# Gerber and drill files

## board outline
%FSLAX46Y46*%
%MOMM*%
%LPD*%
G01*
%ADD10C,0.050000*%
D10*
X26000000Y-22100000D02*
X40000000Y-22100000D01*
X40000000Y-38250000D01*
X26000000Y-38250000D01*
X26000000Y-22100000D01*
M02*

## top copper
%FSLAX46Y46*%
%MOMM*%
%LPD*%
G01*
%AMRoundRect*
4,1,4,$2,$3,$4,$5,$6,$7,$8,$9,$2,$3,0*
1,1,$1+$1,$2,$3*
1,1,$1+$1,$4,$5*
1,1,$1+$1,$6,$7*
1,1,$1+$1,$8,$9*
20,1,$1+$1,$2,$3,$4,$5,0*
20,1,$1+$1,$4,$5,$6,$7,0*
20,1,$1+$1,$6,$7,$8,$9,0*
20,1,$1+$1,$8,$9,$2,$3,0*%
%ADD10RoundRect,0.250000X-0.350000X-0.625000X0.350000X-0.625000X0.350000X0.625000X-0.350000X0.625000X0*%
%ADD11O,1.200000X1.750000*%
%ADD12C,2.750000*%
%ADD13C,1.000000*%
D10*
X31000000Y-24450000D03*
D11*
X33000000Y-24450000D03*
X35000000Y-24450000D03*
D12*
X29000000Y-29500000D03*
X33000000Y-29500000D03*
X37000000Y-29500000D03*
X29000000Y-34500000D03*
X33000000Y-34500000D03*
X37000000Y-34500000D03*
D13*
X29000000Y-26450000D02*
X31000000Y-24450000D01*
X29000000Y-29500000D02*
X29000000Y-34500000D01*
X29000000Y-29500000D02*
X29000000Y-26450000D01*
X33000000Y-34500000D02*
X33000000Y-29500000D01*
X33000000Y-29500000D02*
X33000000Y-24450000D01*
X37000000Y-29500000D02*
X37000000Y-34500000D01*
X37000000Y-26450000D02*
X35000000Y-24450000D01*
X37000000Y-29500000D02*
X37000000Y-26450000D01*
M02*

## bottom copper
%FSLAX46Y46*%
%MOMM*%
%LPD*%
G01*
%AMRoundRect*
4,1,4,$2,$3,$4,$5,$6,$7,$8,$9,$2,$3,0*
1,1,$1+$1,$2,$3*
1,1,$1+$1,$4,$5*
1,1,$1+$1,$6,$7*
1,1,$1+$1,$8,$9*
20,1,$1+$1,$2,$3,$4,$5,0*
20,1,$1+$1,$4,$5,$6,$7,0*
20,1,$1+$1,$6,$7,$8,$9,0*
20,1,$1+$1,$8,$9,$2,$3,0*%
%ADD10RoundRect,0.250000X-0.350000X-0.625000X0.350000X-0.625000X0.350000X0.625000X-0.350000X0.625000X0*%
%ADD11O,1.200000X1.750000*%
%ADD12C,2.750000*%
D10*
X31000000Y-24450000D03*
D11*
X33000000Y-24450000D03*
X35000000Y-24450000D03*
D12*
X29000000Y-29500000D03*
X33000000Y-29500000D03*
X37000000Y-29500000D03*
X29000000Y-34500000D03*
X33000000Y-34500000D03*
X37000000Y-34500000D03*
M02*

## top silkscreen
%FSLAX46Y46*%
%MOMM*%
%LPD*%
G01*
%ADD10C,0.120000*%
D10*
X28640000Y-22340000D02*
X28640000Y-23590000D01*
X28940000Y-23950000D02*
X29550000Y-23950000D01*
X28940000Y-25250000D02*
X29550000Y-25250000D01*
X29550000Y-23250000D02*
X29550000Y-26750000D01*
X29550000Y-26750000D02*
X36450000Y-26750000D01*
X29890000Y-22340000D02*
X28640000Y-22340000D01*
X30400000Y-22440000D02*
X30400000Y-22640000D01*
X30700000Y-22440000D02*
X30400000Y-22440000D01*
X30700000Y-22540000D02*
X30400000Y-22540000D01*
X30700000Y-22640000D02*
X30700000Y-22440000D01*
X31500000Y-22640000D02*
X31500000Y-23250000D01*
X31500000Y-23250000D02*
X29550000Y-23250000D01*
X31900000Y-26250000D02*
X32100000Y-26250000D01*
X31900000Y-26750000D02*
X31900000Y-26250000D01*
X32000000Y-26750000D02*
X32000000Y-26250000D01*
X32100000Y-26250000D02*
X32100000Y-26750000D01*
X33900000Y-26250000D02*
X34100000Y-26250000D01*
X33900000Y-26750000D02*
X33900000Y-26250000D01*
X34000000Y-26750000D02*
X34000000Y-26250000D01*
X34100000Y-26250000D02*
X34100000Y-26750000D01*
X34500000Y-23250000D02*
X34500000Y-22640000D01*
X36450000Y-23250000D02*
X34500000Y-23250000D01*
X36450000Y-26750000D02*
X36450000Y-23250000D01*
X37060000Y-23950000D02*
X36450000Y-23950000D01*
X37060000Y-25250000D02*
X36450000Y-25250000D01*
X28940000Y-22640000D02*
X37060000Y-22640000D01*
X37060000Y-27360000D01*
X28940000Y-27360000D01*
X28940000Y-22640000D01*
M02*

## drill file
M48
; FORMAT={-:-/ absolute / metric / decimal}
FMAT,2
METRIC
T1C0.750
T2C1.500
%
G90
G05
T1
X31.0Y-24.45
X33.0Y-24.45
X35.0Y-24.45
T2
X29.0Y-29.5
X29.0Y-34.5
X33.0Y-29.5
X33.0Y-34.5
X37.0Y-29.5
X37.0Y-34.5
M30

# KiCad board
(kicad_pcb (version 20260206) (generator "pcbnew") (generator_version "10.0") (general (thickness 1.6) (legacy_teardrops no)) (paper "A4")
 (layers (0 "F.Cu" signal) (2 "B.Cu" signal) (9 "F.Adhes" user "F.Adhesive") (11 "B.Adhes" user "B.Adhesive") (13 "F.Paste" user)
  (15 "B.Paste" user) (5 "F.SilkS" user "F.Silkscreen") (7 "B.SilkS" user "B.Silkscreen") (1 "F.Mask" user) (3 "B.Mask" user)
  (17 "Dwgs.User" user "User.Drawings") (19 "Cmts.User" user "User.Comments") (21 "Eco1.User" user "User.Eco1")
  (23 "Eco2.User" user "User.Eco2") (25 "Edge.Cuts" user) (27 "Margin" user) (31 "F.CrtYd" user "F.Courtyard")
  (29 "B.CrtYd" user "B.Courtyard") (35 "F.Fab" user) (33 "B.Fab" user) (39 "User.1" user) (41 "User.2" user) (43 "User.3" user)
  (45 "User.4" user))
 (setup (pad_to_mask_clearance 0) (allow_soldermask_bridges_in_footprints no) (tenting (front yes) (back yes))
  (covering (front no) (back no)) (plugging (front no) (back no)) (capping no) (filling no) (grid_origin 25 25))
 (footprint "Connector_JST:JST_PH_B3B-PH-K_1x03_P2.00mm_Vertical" (layer "F.Cu") (at 31 24.45)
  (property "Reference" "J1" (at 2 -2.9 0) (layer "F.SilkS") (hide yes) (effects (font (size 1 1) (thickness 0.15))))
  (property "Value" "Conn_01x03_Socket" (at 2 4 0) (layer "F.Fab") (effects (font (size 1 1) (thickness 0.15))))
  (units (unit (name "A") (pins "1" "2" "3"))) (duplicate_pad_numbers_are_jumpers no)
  (fp_line (start -2.36 -2.11) (end -2.36 -0.86) (stroke (width 0.12) (type solid)) (layer "F.SilkS"))
  (fp_line (start -2.06 -0.5) (end -1.45 -0.5) (stroke (width 0.12) (type solid)) (layer "F.SilkS"))
  (fp_line (start -2.06 0.8) (end -1.45 0.8) (stroke (width 0.12) (type solid)) (layer "F.SilkS"))
  (fp_line (start -1.45 -1.2) (end -1.45 2.3) (stroke (width 0.12) (type solid)) (layer "F.SilkS"))
  (fp_line (start -1.45 2.3) (end 5.45 2.3) (stroke (width 0.12) (type solid)) (layer "F.SilkS"))
  (fp_line (start -1.11 -2.11) (end -2.36 -2.11) (stroke (width 0.12) (type solid)) (layer "F.SilkS"))
  (fp_line (start -0.6 -2.01) (end -0.6 -1.81) (stroke (width 0.12) (type solid)) (layer "F.SilkS"))
  (fp_line (start -0.3 -2.01) (end -0.6 -2.01) (stroke (width 0.12) (type solid)) (layer "F.SilkS"))
  (fp_line (start -0.3 -1.91) (end -0.6 -1.91) (stroke (width 0.12) (type solid)) (layer "F.SilkS"))
  (fp_line (start -0.3 -1.81) (end -0.3 -2.01) (stroke (width 0.12) (type solid)) (layer "F.SilkS"))
  (fp_line (start 0.5 -1.81) (end 0.5 -1.2) (stroke (width 0.12) (type solid)) (layer "F.SilkS"))
  (fp_line (start 0.5 -1.2) (end -1.45 -1.2) (stroke (width 0.12) (type solid)) (layer "F.SilkS"))
  (fp_line (start 0.9 1.8) (end 1.1 1.8) (stroke (width 0.12) (type solid)) (layer "F.SilkS"))
  (fp_line (start 0.9 2.3) (end 0.9 1.8) (stroke (width 0.12) (type solid)) (layer "F.SilkS"))
  (fp_line (start 1 2.3) (end 1 1.8) (stroke (width 0.12) (type solid)) (layer "F.SilkS"))
  (fp_line (start 1.1 1.8) (end 1.1 2.3) (stroke (width 0.12) (type solid)) (layer "F.SilkS"))
  (fp_line (start 2.9 1.8) (end 3.1 1.8) (stroke (width 0.12) (type solid)) (layer "F.SilkS"))
  (fp_line (start 2.9 2.3) (end 2.9 1.8) (stroke (width 0.12) (type solid)) (layer "F.SilkS"))
  (fp_line (start 3 2.3) (end 3 1.8) (stroke (width 0.12) (type solid)) (layer "F.SilkS"))
  (fp_line (start 3.1 1.8) (end 3.1 2.3) (stroke (width 0.12) (type solid)) (layer "F.SilkS"))
  (fp_line (start 3.5 -1.2) (end 3.5 -1.81) (stroke (width 0.12) (type solid)) (layer "F.SilkS"))
  (fp_line (start 5.45 -1.2) (end 3.5 -1.2) (stroke (width 0.12) (type solid)) (layer "F.SilkS"))
  (fp_line (start 5.45 2.3) (end 5.45 -1.2) (stroke (width 0.12) (type solid)) (layer "F.SilkS"))
  (fp_line (start 6.06 -0.5) (end 5.45 -0.5) (stroke (width 0.12) (type solid)) (layer "F.SilkS"))
  (fp_line (start 6.06 0.8) (end 5.45 0.8) (stroke (width 0.12) (type solid)) (layer "F.SilkS"))
  (fp_rect (start -2.06 -1.81) (end 6.06 2.91) (stroke (width 0.12) (type solid)) (fill no) (layer "F.SilkS"))
  (pad "1" thru_hole roundrect (at 0 0) (size 1.2 1.75) (drill 0.75) (layers "*.Cu" "*.Mask") (remove_unused_layers no)
   (roundrect_rratio 0.208333) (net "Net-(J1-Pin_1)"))
  (pad "2" thru_hole oval (at 2 0) (size 1.2 1.75) (drill 0.75) (layers "*.Cu" "*.Mask") (remove_unused_layers no) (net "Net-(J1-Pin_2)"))
  (pad "3" thru_hole oval (at 4 0) (size 1.2 1.75) (drill 0.75) (layers "*.Cu" "*.Mask") (remove_unused_layers no) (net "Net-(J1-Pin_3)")))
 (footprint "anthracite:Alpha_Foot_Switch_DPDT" (layer "B.Cu") (at 33 32 180)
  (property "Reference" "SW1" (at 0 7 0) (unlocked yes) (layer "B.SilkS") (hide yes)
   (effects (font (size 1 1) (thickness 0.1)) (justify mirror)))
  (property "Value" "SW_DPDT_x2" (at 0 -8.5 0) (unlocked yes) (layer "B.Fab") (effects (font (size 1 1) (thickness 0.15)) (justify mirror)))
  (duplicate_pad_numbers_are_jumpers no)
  (pad "1" thru_hole circle (at 4 2.5 180) (size 2.75 2.75) (drill 1.5) (layers "*.Cu" "*.Mask") (remove_unused_layers no)
   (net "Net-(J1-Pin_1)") (zone_connect 2))
  (pad "2" thru_hole circle (at 0 2.5 180) (size 2.75 2.75) (drill 1.5) (layers "*.Cu" "*.Mask") (remove_unused_layers no)
   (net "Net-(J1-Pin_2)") (zone_connect 2))
  (pad "3" thru_hole circle (at -4 2.5 180) (size 2.75 2.75) (drill 1.5) (layers "*.Cu" "*.Mask") (remove_unused_layers no)
   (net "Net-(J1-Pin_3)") (zone_connect 2))
  (pad "4" thru_hole circle (at 4 -2.5 180) (size 2.75 2.75) (drill 1.5) (layers "*.Cu" "*.Mask") (remove_unused_layers no)
   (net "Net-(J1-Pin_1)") (zone_connect 2))
  (pad "5" thru_hole circle (at 0 -2.5 180) (size 2.75 2.75) (drill 1.5) (layers "*.Cu" "*.Mask") (remove_unused_layers no)
   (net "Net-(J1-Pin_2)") (zone_connect 2))
  (pad "6" thru_hole circle (at -4 -2.5 180) (size 2.75 2.75) (drill 1.5) (layers "*.Cu" "*.Mask") (remove_unused_layers no)
   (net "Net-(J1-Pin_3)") (zone_connect 2)))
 (gr_rect (start 26 22.1) (end 40 38.25) (stroke (width 0.05) (type default)) (fill no) (layer "Edge.Cuts"))
 (segment (start 29 26.45) (end 31 24.45) (width 1) (layer "F.Cu") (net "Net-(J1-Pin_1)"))
 (segment (start 29 29.5) (end 29 34.5) (width 1) (layer "F.Cu") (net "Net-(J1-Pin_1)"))
 (segment (start 29 29.5) (end 29 26.45) (width 1) (layer "F.Cu") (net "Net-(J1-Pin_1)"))
 (segment (start 33 34.5) (end 33 29.5) (width 1) (layer "F.Cu") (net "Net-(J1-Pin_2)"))
 (segment (start 33 29.5) (end 33 24.45) (width 1) (layer "F.Cu") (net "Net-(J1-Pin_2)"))
 (segment (start 37 29.5) (end 37 34.5) (width 1) (layer "F.Cu") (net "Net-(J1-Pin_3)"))
 (segment (start 37 26.45) (end 35 24.45) (width 1) (layer "F.Cu") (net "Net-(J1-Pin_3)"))
 (segment (start 37 29.5) (end 37 26.45) (width 1) (layer "F.Cu") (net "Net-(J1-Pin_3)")))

